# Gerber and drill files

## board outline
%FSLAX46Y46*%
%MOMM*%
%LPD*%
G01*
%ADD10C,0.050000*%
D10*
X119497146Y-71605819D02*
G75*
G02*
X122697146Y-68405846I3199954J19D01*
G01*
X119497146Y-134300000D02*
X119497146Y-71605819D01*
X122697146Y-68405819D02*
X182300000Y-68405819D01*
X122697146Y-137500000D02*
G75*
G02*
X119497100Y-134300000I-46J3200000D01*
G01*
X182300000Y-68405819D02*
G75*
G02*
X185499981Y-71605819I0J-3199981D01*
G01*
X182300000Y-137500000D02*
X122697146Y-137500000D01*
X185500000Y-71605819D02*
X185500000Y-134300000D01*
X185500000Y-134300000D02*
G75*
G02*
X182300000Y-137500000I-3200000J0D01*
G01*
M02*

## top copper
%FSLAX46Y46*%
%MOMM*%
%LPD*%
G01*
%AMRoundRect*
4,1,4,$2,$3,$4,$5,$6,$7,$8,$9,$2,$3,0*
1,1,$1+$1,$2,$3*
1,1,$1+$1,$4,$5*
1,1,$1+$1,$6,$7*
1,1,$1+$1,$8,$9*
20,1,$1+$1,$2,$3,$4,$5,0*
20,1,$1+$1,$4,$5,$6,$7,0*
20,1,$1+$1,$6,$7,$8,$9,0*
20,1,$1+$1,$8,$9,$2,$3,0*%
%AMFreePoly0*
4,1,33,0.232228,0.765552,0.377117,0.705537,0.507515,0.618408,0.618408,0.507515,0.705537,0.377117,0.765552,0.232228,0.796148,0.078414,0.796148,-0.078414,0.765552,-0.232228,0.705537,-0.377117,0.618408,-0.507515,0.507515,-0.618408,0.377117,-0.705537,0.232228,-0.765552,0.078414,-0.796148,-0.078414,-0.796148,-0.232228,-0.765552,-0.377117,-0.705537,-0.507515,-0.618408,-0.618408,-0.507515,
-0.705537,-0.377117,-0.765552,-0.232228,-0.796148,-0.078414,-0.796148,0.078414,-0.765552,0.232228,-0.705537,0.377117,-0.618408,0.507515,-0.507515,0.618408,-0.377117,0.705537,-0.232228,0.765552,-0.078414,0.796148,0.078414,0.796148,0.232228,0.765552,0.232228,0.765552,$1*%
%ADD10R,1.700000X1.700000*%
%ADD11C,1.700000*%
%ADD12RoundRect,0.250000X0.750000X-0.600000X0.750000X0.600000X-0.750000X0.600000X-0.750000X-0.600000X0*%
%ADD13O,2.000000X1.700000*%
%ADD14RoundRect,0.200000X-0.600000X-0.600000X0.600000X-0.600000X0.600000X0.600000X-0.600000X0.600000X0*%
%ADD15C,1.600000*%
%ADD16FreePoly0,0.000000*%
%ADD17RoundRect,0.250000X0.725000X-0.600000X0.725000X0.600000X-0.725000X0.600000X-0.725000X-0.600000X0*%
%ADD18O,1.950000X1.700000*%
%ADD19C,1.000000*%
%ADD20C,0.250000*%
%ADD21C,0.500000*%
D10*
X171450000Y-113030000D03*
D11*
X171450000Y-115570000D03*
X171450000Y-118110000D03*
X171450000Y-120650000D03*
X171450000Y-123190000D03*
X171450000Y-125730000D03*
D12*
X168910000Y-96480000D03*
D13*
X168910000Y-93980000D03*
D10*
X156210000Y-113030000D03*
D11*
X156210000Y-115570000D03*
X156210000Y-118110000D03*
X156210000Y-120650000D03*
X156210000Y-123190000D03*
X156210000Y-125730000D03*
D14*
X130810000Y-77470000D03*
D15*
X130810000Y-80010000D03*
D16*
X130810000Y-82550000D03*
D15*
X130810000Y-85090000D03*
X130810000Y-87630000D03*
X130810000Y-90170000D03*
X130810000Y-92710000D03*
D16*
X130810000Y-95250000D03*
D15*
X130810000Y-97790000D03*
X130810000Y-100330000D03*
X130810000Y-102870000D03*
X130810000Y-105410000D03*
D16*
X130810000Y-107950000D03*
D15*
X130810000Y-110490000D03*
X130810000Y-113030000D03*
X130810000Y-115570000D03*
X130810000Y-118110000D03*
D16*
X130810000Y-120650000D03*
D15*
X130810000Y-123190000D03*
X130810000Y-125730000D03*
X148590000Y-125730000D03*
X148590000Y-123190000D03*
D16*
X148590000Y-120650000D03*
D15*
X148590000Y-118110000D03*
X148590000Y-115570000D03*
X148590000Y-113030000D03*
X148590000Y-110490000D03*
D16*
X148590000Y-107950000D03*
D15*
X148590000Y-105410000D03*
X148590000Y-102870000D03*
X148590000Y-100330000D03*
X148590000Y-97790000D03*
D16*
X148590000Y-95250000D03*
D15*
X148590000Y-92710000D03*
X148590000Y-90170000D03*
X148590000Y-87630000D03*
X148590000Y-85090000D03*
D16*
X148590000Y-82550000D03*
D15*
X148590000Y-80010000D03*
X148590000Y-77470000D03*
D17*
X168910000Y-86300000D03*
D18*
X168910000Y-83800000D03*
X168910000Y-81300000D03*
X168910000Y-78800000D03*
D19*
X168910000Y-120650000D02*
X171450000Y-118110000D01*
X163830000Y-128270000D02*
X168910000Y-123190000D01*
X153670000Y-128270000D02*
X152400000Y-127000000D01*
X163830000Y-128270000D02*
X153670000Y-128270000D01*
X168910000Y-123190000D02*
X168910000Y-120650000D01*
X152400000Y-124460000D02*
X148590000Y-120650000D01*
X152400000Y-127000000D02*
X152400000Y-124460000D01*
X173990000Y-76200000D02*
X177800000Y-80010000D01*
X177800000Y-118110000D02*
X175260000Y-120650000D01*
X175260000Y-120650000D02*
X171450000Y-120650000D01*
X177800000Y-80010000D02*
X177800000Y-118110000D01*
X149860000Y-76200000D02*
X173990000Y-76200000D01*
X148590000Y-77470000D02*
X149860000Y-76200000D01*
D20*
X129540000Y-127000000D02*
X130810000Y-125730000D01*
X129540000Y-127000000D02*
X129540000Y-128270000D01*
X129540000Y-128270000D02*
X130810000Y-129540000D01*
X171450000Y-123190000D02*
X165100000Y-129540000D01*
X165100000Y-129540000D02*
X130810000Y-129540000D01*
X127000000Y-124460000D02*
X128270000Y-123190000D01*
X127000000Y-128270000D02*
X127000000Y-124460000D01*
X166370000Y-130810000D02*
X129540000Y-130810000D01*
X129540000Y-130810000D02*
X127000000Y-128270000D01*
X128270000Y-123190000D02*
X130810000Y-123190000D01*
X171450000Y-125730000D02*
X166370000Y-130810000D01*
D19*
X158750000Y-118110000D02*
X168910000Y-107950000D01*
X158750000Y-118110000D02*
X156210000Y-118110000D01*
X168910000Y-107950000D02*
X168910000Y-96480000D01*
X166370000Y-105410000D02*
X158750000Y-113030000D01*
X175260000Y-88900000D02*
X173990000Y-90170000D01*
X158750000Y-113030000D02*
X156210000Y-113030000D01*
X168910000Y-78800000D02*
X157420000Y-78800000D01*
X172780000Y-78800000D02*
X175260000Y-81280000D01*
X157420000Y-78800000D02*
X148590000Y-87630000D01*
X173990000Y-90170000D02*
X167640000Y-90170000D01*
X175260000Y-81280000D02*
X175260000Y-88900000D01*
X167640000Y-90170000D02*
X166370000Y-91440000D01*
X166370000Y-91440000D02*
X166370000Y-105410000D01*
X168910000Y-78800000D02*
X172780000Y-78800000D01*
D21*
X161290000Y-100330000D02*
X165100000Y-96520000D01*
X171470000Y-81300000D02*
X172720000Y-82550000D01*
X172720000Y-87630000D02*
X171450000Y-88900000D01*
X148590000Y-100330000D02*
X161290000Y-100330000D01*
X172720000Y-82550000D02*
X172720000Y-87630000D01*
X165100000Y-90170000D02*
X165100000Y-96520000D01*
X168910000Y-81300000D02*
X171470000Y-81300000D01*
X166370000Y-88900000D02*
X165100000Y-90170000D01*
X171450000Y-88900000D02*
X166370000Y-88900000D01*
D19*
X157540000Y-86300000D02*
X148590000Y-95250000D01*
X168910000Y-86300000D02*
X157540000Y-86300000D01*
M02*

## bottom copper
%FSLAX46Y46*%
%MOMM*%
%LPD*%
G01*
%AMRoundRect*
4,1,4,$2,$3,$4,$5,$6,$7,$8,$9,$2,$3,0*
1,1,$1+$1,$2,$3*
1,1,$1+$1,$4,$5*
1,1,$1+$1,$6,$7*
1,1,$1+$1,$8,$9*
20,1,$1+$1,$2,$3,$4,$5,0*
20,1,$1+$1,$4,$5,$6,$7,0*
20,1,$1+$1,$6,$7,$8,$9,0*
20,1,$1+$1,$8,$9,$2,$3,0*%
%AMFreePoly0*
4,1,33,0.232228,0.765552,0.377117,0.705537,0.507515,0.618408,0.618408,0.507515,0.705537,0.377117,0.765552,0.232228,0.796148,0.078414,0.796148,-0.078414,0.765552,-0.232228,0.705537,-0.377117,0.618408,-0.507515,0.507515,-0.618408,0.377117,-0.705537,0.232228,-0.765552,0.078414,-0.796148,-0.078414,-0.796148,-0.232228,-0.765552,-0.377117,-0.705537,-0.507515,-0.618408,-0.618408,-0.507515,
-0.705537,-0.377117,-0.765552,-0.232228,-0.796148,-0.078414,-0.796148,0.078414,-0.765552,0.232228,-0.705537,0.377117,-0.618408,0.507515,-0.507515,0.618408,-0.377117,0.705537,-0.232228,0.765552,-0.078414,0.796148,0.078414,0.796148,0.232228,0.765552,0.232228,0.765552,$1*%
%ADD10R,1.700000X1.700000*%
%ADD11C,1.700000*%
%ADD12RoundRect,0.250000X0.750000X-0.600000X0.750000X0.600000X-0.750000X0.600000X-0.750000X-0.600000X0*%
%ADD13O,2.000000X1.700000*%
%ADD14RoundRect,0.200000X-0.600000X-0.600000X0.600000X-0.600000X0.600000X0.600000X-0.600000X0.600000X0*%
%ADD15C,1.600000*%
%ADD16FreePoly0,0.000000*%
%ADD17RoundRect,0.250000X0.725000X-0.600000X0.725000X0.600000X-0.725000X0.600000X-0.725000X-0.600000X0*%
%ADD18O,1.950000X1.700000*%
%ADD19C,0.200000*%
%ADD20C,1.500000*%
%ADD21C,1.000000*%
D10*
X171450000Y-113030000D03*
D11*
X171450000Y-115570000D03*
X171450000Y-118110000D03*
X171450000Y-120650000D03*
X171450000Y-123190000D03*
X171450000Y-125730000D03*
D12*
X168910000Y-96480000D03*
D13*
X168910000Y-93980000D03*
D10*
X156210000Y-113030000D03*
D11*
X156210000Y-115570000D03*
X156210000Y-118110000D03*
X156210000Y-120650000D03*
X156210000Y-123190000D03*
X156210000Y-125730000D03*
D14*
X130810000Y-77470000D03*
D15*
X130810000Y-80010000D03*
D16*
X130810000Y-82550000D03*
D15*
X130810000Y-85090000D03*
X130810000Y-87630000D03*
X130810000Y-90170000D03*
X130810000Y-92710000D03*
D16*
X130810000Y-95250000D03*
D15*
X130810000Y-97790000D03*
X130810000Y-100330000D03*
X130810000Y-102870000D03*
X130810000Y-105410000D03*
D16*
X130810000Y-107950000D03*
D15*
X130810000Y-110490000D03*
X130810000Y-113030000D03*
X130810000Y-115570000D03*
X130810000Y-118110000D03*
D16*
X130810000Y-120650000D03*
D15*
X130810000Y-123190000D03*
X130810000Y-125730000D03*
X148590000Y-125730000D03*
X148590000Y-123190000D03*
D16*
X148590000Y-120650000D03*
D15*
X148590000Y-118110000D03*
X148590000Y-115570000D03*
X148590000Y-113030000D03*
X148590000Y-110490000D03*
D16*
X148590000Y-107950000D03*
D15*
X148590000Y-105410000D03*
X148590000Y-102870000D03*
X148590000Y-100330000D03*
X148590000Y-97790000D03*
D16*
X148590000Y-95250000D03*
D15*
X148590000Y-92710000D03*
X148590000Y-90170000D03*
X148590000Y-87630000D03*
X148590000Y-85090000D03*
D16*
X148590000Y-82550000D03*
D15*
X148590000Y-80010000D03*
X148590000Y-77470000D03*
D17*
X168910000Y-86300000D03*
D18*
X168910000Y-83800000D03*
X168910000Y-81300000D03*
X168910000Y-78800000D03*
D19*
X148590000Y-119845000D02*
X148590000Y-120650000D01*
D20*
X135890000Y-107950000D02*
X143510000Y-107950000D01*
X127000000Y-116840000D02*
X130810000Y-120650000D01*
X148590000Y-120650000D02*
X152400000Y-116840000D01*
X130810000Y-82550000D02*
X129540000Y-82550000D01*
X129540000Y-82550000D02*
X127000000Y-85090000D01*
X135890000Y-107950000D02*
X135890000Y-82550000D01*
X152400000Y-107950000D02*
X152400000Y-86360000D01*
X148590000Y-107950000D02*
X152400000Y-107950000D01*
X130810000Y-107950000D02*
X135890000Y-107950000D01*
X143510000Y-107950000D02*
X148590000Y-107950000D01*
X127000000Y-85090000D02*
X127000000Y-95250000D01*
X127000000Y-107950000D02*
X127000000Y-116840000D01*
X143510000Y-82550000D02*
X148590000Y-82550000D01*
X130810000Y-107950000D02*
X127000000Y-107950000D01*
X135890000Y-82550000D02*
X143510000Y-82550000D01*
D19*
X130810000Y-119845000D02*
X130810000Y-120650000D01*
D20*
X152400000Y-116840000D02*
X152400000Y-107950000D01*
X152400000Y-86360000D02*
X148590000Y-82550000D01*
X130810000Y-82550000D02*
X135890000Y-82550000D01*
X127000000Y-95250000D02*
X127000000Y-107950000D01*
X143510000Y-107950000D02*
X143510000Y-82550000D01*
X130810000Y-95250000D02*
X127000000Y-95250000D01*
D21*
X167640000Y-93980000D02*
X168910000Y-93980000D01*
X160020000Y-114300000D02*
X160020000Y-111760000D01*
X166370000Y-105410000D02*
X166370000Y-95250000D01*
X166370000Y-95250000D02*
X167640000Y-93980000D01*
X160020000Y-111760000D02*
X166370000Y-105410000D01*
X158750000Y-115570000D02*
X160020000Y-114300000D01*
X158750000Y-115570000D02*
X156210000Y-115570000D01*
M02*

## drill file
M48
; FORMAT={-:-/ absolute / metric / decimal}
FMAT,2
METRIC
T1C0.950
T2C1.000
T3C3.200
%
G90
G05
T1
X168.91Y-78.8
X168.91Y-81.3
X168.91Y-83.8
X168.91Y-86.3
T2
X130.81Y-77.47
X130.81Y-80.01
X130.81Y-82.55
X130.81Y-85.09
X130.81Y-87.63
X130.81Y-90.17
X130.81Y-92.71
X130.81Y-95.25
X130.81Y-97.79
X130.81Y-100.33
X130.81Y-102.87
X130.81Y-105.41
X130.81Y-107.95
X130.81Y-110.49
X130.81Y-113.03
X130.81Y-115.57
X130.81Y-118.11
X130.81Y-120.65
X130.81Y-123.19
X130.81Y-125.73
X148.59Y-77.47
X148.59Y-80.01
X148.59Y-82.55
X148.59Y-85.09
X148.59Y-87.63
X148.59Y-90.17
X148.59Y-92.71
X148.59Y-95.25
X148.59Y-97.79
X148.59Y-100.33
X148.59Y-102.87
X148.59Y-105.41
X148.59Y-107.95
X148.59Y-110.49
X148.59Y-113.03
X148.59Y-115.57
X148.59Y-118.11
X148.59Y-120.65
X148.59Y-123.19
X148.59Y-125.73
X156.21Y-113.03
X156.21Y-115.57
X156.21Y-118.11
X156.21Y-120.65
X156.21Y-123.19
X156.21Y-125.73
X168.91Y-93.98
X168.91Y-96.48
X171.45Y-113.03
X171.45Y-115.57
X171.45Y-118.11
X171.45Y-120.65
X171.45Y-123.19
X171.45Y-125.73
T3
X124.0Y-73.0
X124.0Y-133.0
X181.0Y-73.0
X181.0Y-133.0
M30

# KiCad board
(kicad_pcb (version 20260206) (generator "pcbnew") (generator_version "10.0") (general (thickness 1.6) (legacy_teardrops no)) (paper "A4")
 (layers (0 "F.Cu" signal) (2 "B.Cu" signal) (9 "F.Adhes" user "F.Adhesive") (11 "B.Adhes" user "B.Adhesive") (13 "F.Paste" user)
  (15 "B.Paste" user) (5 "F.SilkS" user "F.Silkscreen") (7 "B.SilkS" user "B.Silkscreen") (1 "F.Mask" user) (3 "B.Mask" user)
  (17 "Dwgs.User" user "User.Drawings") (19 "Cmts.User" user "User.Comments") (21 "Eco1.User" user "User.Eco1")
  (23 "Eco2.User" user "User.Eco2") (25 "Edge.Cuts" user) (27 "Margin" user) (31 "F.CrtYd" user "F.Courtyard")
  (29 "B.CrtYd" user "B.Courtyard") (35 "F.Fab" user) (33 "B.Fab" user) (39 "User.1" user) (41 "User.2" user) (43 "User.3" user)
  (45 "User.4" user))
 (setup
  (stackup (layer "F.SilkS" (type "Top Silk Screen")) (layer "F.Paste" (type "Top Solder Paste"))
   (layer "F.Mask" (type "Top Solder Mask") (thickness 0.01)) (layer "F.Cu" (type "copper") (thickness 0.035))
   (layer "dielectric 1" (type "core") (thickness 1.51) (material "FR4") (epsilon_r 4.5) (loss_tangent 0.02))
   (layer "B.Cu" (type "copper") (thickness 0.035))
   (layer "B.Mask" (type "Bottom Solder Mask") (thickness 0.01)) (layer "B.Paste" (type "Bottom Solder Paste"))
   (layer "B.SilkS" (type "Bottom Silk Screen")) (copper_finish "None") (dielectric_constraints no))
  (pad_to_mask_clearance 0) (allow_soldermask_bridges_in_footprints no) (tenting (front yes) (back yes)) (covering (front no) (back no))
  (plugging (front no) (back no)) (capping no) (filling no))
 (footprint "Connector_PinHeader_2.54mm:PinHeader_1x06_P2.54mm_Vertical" (layer "F.Cu") (at 171.45 113.03)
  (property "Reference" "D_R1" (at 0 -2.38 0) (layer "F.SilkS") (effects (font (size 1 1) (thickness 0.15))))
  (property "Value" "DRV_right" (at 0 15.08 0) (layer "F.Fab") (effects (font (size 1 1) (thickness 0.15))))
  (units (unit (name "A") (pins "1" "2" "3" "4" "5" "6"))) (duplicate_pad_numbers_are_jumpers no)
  (pad "1" thru_hole rect (at 0 0) (size 1.7 1.7) (drill 1) (layers "*.Cu" "*.Mask") (remove_unused_layers no) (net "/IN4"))
  (pad "2" thru_hole circle (at 0 2.54) (size 1.7 1.7) (drill 1) (layers "*.Cu" "*.Mask") (remove_unused_layers no) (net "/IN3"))
  (pad "3" thru_hole circle (at 0 5.08) (size 1.7 1.7) (drill 1) (layers "*.Cu" "*.Mask") (remove_unused_layers no) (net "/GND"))
  (pad "4" thru_hole circle (at 0 7.62) (size 1.7 1.7) (drill 1) (layers "*.Cu" "*.Mask") (remove_unused_layers no) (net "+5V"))
  (pad "5" thru_hole circle (at 0 10.16) (size 1.7 1.7) (drill 1) (layers "*.Cu" "*.Mask") (remove_unused_layers no) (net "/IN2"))
  (pad "6" thru_hole circle (at 0 12.7) (size 1.7 1.7) (drill 1) (layers "*.Cu" "*.Mask") (remove_unused_layers no) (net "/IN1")))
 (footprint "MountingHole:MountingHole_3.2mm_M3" (layer "F.Cu") (at 181 133)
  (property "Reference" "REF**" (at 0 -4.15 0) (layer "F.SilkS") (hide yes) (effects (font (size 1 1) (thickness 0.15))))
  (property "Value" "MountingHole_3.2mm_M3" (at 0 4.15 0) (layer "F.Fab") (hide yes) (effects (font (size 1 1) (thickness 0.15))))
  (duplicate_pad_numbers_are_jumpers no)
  (pad "" np_thru_hole circle (at 0 0) (size 3.2 3.2) (drill 3.2) (layers "*.Cu" "*.Mask")))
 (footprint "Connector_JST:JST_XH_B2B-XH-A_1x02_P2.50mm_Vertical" (layer "F.Cu") (at 168.91 96.48 90)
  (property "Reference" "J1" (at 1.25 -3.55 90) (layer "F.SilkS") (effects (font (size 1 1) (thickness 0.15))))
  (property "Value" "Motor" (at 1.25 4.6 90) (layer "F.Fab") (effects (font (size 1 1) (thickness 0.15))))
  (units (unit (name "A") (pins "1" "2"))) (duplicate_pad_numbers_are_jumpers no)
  (pad "1" thru_hole roundrect (at 0 0 90) (size 1.7 2) (drill 1) (layers "*.Cu" "*.Mask") (remove_unused_layers no)
   (roundrect_rratio 0.147059) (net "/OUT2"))
  (pad "2" thru_hole oval (at 2.5 0 90) (size 1.7 2) (drill 1) (layers "*.Cu" "*.Mask") (remove_unused_layers no) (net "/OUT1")))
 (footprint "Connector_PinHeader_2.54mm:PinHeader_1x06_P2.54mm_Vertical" (layer "F.Cu") (at 156.21 113.03)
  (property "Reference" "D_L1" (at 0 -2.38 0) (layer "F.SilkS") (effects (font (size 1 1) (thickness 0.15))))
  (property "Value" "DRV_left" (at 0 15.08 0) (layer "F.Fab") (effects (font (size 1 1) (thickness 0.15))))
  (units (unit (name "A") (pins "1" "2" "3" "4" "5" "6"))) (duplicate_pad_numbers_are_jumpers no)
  (pad "1" thru_hole rect (at 0 0) (size 1.7 1.7) (drill 1) (layers "*.Cu" "*.Mask") (remove_unused_layers no) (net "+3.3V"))
  (pad "2" thru_hole circle (at 0 2.54) (size 1.7 1.7) (drill 1) (layers "*.Cu" "*.Mask") (remove_unused_layers no) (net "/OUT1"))
  (pad "3" thru_hole circle (at 0 5.08) (size 1.7 1.7) (drill 1) (layers "*.Cu" "*.Mask") (remove_unused_layers no) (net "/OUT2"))
  (pad "4" thru_hole circle (at 0 7.62) (size 1.7 1.7) (drill 1) (layers "*.Cu" "*.Mask") (remove_unused_layers no) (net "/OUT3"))
  (pad "5" thru_hole circle (at 0 10.16) (size 1.7 1.7) (drill 1) (layers "*.Cu" "*.Mask") (remove_unused_layers no) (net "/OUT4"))
  (pad "6" thru_hole circle (at 0 12.7) (size 1.7 1.7) (drill 1) (layers "*.Cu" "*.Mask") (remove_unused_layers no) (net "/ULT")))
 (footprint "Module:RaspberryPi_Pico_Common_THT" (layer "F.Cu") (at 130.81 77.47)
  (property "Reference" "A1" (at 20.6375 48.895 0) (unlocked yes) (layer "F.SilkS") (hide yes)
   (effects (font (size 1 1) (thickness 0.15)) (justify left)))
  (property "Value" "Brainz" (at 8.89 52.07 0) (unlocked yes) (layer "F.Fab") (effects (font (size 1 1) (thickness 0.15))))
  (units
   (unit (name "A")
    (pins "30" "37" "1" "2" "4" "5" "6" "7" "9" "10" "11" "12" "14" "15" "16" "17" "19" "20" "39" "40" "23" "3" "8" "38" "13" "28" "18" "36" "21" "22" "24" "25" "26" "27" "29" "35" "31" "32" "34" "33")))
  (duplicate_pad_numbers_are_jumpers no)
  (pad "1" thru_hole roundrect (at 0 0) (size 1.6 1.6) (drill 1) (layers "*.Cu" "*.Mask") (remove_unused_layers no) (roundrect_rratio 0.125)
   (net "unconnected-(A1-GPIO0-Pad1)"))
  (pad "2" thru_hole circle (at 0 2.54) (size 1.6 1.6) (drill 1) (layers "*.Cu" "*.Mask") (remove_unused_layers no)
   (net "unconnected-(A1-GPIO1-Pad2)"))
  (pad "3" thru_hole custom (at 0 5.08) (size 1.6 1.6) (drill 1) (layers "*.Cu" "*.Mask") (remove_unused_layers no) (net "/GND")
   (options (clearance outline) (anchor circle)) (primitives))
  (pad "4" thru_hole circle (at 0 7.62) (size 1.6 1.6) (drill 1) (layers "*.Cu" "*.Mask") (remove_unused_layers no)
   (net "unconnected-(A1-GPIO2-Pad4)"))
  (pad "5" thru_hole circle (at 0 10.16) (size 1.6 1.6) (drill 1) (layers "*.Cu" "*.Mask") (remove_unused_layers no)
   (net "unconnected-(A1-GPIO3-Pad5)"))
  (pad "6" thru_hole circle (at 0 12.7) (size 1.6 1.6) (drill 1) (layers "*.Cu" "*.Mask") (remove_unused_layers no)
   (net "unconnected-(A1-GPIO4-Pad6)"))
  (pad "7" thru_hole circle (at 0 15.24) (size 1.6 1.6) (drill 1) (layers "*.Cu" "*.Mask") (remove_unused_layers no)
   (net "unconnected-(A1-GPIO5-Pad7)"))
  (pad "8" thru_hole custom (at 0 17.78) (size 1.6 1.6) (drill 1) (layers "*.Cu" "*.Mask") (remove_unused_layers no) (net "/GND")
   (options (clearance outline) (anchor circle)) (primitives))
  (pad "9" thru_hole circle (at 0 20.32) (size 1.6 1.6) (drill 1) (layers "*.Cu" "*.Mask") (remove_unused_layers no)
   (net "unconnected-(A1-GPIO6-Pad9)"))
  (pad "10" thru_hole circle (at 0 22.86) (size 1.6 1.6) (drill 1) (layers "*.Cu" "*.Mask") (remove_unused_layers no)
   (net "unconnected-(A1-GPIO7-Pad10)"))
  (pad "11" thru_hole circle (at 0 25.4) (size 1.6 1.6) (drill 1) (layers "*.Cu" "*.Mask") (remove_unused_layers no)
   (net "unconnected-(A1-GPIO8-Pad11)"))
  (pad "12" thru_hole circle (at 0 27.94) (size 1.6 1.6) (drill 1) (layers "*.Cu" "*.Mask") (remove_unused_layers no)
   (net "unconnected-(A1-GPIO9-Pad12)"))
  (pad "13" thru_hole custom (at 0 30.48) (size 1.6 1.6) (drill 1) (layers "*.Cu" "*.Mask") (remove_unused_layers no) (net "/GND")
   (options (clearance outline) (anchor circle)) (primitives))
  (pad "14" thru_hole circle (at 0 33.02) (size 1.6 1.6) (drill 1) (layers "*.Cu" "*.Mask") (remove_unused_layers no)
   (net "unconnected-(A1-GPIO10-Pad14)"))
  (pad "15" thru_hole circle (at 0 35.56) (size 1.6 1.6) (drill 1) (layers "*.Cu" "*.Mask") (remove_unused_layers no)
   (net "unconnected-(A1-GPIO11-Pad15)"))
  (pad "16" thru_hole circle (at 0 38.1) (size 1.6 1.6) (drill 1) (layers "*.Cu" "*.Mask") (remove_unused_layers no)
   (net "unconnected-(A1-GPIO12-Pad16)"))
  (pad "17" thru_hole circle (at 0 40.64) (size 1.6 1.6) (drill 1) (layers "*.Cu" "*.Mask") (remove_unused_layers no)
   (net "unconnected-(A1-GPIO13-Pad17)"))
  (pad "18" thru_hole custom (at 0 43.18) (size 1.6 1.6) (drill 1) (layers "*.Cu" "*.Mask") (remove_unused_layers no) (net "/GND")
   (options (clearance outline) (anchor circle)) (primitives))
  (pad "19" thru_hole circle (at 0 45.72) (size 1.6 1.6) (drill 1) (layers "*.Cu" "*.Mask") (remove_unused_layers no) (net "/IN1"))
  (pad "20" thru_hole circle (at 0 48.26) (size 1.6 1.6) (drill 1) (layers "*.Cu" "*.Mask") (remove_unused_layers no) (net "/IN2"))
  (pad "21" thru_hole circle (at 17.78 48.26) (size 1.6 1.6) (drill 1) (layers "*.Cu" "*.Mask") (remove_unused_layers no)
   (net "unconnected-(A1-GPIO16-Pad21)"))
  (pad "22" thru_hole circle (at 17.78 45.72) (size 1.6 1.6) (drill 1) (layers "*.Cu" "*.Mask") (remove_unused_layers no)
   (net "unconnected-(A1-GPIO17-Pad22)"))
  (pad "23" thru_hole custom (at 17.78 43.18) (size 1.6 1.6) (drill 1) (layers "*.Cu" "*.Mask") (remove_unused_layers no) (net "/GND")
   (options (clearance outline) (anchor circle)) (primitives))
  (pad "24" thru_hole circle (at 17.78 40.64) (size 1.6 1.6) (drill 1) (layers "*.Cu" "*.Mask") (remove_unused_layers no)
   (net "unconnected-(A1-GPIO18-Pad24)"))
  (pad "25" thru_hole circle (at 17.78 38.1) (size 1.6 1.6) (drill 1) (layers "*.Cu" "*.Mask") (remove_unused_layers no)
   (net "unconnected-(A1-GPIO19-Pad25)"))
  (pad "26" thru_hole circle (at 17.78 35.56) (size 1.6 1.6) (drill 1) (layers "*.Cu" "*.Mask") (remove_unused_layers no)
   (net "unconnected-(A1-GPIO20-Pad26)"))
  (pad "27" thru_hole circle (at 17.78 33.02) (size 1.6 1.6) (drill 1) (layers "*.Cu" "*.Mask") (remove_unused_layers no)
   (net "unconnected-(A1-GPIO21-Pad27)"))
  (pad "28" thru_hole custom (at 17.78 30.48) (size 1.6 1.6) (drill 1) (layers "*.Cu" "*.Mask") (remove_unused_layers no) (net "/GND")
   (options (clearance outline) (anchor circle)) (primitives))
  (pad "29" thru_hole circle (at 17.78 27.94) (size 1.6 1.6) (drill 1) (layers "*.Cu" "*.Mask") (remove_unused_layers no)
   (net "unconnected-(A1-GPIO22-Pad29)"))
  (pad "30" thru_hole circle (at 17.78 25.4) (size 1.6 1.6) (drill 1) (layers "*.Cu" "*.Mask") (remove_unused_layers no)
   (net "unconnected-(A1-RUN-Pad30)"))
  (pad "31" thru_hole circle (at 17.78 22.86) (size 1.6 1.6) (drill 1) (layers "*.Cu" "*.Mask") (remove_unused_layers no) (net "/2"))
  (pad "32" thru_hole circle (at 17.78 20.32) (size 1.6 1.6) (drill 1) (layers "*.Cu" "*.Mask") (remove_unused_layers no)
   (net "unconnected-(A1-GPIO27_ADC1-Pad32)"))
  (pad "33" thru_hole custom (at 17.78 17.78) (size 1.6 1.6) (drill 1) (layers "*.Cu" "*.Mask") (remove_unused_layers no) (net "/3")
   (options (clearance outline) (anchor circle)) (primitives))
  (pad "34" thru_hole circle (at 17.78 15.24) (size 1.6 1.6) (drill 1) (layers "*.Cu" "*.Mask") (remove_unused_layers no)
   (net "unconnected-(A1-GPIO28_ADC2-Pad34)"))
  (pad "35" thru_hole circle (at 17.78 12.7) (size 1.6 1.6) (drill 1) (layers "*.Cu" "*.Mask") (remove_unused_layers no)
   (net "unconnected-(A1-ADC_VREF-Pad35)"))
  (pad "36" thru_hole circle (at 17.78 10.16) (size 1.6 1.6) (drill 1) (layers "*.Cu" "*.Mask") (remove_unused_layers no) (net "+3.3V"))
  (pad "37" thru_hole circle (at 17.78 7.62) (size 1.6 1.6) (drill 1) (layers "*.Cu" "*.Mask") (remove_unused_layers no)
   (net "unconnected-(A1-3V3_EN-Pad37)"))
  (pad "38" thru_hole custom (at 17.78 5.08) (size 1.6 1.6) (drill 1) (layers "*.Cu" "*.Mask") (remove_unused_layers no) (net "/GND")
   (options (clearance outline) (anchor circle)) (primitives))
  (pad "39" thru_hole circle (at 17.78 2.54) (size 1.6 1.6) (drill 1) (layers "*.Cu" "*.Mask") (remove_unused_layers no)
   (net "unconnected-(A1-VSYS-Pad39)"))
  (pad "40" thru_hole circle (at 17.78 0) (size 1.6 1.6) (drill 1) (layers "*.Cu" "*.Mask") (remove_unused_layers no) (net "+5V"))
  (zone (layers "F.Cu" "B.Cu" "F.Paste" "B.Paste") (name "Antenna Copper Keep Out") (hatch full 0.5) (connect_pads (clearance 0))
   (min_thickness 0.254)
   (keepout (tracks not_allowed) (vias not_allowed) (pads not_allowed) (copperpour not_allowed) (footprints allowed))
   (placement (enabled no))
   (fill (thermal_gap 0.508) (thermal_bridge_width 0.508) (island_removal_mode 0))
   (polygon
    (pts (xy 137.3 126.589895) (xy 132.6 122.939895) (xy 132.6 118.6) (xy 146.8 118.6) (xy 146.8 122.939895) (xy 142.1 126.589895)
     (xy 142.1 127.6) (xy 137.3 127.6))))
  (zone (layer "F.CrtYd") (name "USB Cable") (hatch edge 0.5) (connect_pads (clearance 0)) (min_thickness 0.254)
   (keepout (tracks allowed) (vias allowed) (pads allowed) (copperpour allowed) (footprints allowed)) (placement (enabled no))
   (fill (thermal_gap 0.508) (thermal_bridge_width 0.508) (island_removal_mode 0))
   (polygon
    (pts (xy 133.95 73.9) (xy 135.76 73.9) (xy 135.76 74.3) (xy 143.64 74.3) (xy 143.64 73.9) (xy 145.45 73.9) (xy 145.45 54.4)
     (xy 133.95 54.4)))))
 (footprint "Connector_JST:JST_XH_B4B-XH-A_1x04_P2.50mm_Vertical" (layer "F.Cu") (at 168.91 86.3 90)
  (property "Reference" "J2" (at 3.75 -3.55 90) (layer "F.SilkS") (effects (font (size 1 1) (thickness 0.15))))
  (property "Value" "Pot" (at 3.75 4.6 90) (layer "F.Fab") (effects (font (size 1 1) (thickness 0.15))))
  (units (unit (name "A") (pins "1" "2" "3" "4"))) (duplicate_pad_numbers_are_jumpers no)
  (pad "1" thru_hole roundrect (at 0 0 90) (size 1.7 1.95) (drill 0.95) (layers "*.Cu" "*.Mask") (remove_unused_layers no)
   (roundrect_rratio 0.147059) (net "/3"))
  (pad "2" thru_hole oval (at 2.5 0 90) (size 1.7 1.95) (drill 0.95) (layers "*.Cu" "*.Mask") (remove_unused_layers no) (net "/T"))
  (pad "3" thru_hole oval (at 5 0 90) (size 1.7 1.95) (drill 0.95) (layers "*.Cu" "*.Mask") (remove_unused_layers no) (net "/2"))
  (pad "4" thru_hole oval (at 7.5 0 90) (size 1.7 1.95) (drill 0.95) (layers "*.Cu" "*.Mask") (remove_unused_layers no) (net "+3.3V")))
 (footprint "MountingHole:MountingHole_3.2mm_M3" (layer "F.Cu") (at 124 133)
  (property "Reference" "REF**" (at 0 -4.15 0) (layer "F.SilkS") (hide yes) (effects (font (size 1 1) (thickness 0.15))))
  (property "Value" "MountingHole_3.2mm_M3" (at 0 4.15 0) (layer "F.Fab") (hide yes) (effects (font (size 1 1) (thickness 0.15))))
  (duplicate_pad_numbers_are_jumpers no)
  (pad "" np_thru_hole circle (at 0 0) (size 3.2 3.2) (drill 3.2) (layers "*.Cu" "*.Mask")))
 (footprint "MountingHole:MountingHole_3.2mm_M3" (layer "F.Cu") (at 124 73)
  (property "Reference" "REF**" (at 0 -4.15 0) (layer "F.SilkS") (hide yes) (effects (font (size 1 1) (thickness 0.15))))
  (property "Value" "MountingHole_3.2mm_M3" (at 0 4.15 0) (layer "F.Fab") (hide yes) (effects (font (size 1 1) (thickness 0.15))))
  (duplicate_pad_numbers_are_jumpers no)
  (pad "" np_thru_hole circle (at 0 0) (size 3.2 3.2) (drill 3.2) (layers "*.Cu" "*.Mask")))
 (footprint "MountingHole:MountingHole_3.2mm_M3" (layer "F.Cu") (at 181 73)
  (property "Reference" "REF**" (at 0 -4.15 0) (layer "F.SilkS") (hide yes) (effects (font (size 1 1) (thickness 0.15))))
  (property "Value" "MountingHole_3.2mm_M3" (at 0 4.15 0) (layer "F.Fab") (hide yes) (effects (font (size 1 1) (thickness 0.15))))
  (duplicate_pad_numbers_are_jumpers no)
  (pad "" np_thru_hole circle (at 0 0) (size 3.2 3.2) (drill 3.2) (layers "*.Cu" "*.Mask")))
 (gr_arc (start 119.497146 71.605819) (mid 120.434404 69.343077) (end 122.697146 68.405819) (stroke (width 0.05) (type default))
  (layer "Edge.Cuts"))
 (gr_line (start 119.497146 134.3) (end 119.497146 71.605819) (stroke (width 0.05) (type default)) (layer "Edge.Cuts"))
 (gr_line (start 122.697146 68.405819) (end 182.3 68.405819) (stroke (width 0.05) (type default)) (layer "Edge.Cuts"))
 (gr_arc (start 122.697146 137.5) (mid 120.434404 136.562742) (end 119.497146 134.3) (stroke (width 0.05) (type default))
  (layer "Edge.Cuts"))
 (gr_arc (start 182.3 68.405819) (mid 184.562735 69.343078) (end 185.5 71.605819) (stroke (width 0.05) (type default)) (layer "Edge.Cuts"))
 (gr_line (start 182.3 137.5) (end 122.697146 137.5) (stroke (width 0.05) (type default)) (layer "Edge.Cuts"))
 (gr_line (start 185.5 71.605819) (end 185.5 134.3) (stroke (width 0.05) (type default)) (layer "Edge.Cuts"))
 (gr_arc (start 185.5 134.3) (mid 184.562742 136.562742) (end 182.3 137.5) (stroke (width 0.05) (type default)) (layer "Edge.Cuts"))
 (segment (start 168.91 120.65) (end 171.45 118.11) (width 1) (layer "F.Cu") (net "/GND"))
 (segment (start 163.83 128.27) (end 168.91 123.19) (width 1) (layer "F.Cu") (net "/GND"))
 (segment (start 153.67 128.27) (end 152.4 127) (width 1) (layer "F.Cu") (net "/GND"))
 (segment (start 163.83 128.27) (end 153.67 128.27) (width 1) (layer "F.Cu") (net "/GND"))
 (segment (start 168.91 123.19) (end 168.91 120.65) (width 1) (layer "F.Cu") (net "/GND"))
 (segment (start 152.4 124.46) (end 148.59 120.65) (width 1) (layer "F.Cu") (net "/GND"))
 (segment (start 152.4 127) (end 152.4 124.46) (width 1) (layer "F.Cu") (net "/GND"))
 (segment (start 148.59 119.845) (end 148.59 120.65) (width 0.2) (layer "B.Cu") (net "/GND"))
 (segment (start 135.89 107.95) (end 143.51 107.95) (width 1.5) (layer "B.Cu") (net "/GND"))
 (segment (start 127 116.84) (end 130.81 120.65) (width 1.5) (layer "B.Cu") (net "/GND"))
 (segment (start 148.59 120.65) (end 152.4 116.84) (width 1.5) (layer "B.Cu") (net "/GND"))
 (segment (start 130.81 82.55) (end 129.54 82.55) (width 1.5) (layer "B.Cu") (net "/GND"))
 (segment (start 129.54 82.55) (end 127 85.09) (width 1.5) (layer "B.Cu") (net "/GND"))
 (segment (start 135.89 107.95) (end 135.89 82.55) (width 1.5) (layer "B.Cu") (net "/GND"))
 (segment (start 152.4 107.95) (end 152.4 86.36) (width 1.5) (layer "B.Cu") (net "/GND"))
 (segment (start 148.59 107.95) (end 152.4 107.95) (width 1.5) (layer "B.Cu") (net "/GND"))
 (segment (start 130.81 107.95) (end 135.89 107.95) (width 1.5) (layer "B.Cu") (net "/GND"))
 (segment (start 143.51 107.95) (end 148.59 107.95) (width 1.5) (layer "B.Cu") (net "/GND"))
 (segment (start 127 85.09) (end 127 95.25) (width 1.5) (layer "B.Cu") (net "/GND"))
 (segment (start 127 107.95) (end 127 116.84) (width 1.5) (layer "B.Cu") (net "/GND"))
 (segment (start 143.51 82.55) (end 148.59 82.55) (width 1.5) (layer "B.Cu") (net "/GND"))
 (segment (start 130.81 107.95) (end 127 107.95) (width 1.5) (layer "B.Cu") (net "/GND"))
 (segment (start 135.89 82.55) (end 143.51 82.55) (width 1.5) (layer "B.Cu") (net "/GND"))
 (segment (start 130.81 119.845) (end 130.81 120.65) (width 0.2) (layer "B.Cu") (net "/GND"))
 (segment (start 152.4 116.84) (end 152.4 107.95) (width 1.5) (layer "B.Cu") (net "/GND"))
 (segment (start 152.4 86.36) (end 148.59 82.55) (width 1.5) (layer "B.Cu") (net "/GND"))
 (segment (start 130.81 82.55) (end 135.89 82.55) (width 1.5) (layer "B.Cu") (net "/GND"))
 (segment (start 127 95.25) (end 127 107.95) (width 1.5) (layer "B.Cu") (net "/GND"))
 (segment (start 143.51 107.95) (end 143.51 82.55) (width 1.5) (layer "B.Cu") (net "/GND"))
 (segment (start 130.81 95.25) (end 127 95.25) (width 1.5) (layer "B.Cu") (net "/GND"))
 (segment (start 173.99 76.2) (end 177.8 80.01) (width 1) (layer "F.Cu") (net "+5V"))
 (segment (start 177.8 118.11) (end 175.26 120.65) (width 1) (layer "F.Cu") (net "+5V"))
 (segment (start 175.26 120.65) (end 171.45 120.65) (width 1) (layer "F.Cu") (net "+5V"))
 (segment (start 177.8 80.01) (end 177.8 118.11) (width 1) (layer "F.Cu") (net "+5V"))
 (segment (start 149.86 76.2) (end 173.99 76.2) (width 1) (layer "F.Cu") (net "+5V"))
 (segment (start 148.59 77.47) (end 149.86 76.2) (width 1) (layer "F.Cu") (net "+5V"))
 (segment (start 129.54 127) (end 130.81 125.73) (width 0.25) (layer "F.Cu") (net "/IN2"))
 (segment (start 129.54 127) (end 129.54 128.27) (width 0.25) (layer "F.Cu") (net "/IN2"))
 (segment (start 129.54 128.27) (end 130.81 129.54) (width 0.25) (layer "F.Cu") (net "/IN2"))
 (segment (start 171.45 123.19) (end 165.1 129.54) (width 0.25) (layer "F.Cu") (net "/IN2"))
 (segment (start 165.1 129.54) (end 130.81 129.54) (width 0.25) (layer "F.Cu") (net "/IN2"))
 (segment (start 127 124.46) (end 128.27 123.19) (width 0.25) (layer "F.Cu") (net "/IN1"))
 (segment (start 127 128.27) (end 127 124.46) (width 0.25) (layer "F.Cu") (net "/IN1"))
 (segment (start 166.37 130.81) (end 129.54 130.81) (width 0.25) (layer "F.Cu") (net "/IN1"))
 (segment (start 129.54 130.81) (end 127 128.27) (width 0.25) (layer "F.Cu") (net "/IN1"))
 (segment (start 128.27 123.19) (end 130.81 123.19) (width 0.25) (layer "F.Cu") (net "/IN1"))
 (segment (start 171.45 125.73) (end 166.37 130.81) (width 0.25) (layer "F.Cu") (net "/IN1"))
 (segment (start 158.75 118.11) (end 168.91 107.95) (width 1) (layer "F.Cu") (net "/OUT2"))
 (segment (start 158.75 118.11) (end 156.21 118.11) (width 1) (layer "F.Cu") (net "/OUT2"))
 (segment (start 168.91 107.95) (end 168.91 96.48) (width 1) (layer "F.Cu") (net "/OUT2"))
 (segment (start 167.64 93.98) (end 168.91 93.98) (width 1) (layer "B.Cu") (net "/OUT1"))
 (segment (start 160.02 114.3) (end 160.02 111.76) (width 1) (layer "B.Cu") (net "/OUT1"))
 (segment (start 166.37 105.41) (end 166.37 95.25) (width 1) (layer "B.Cu") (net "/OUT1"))
 (segment (start 166.37 95.25) (end 167.64 93.98) (width 1) (layer "B.Cu") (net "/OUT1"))
 (segment (start 160.02 111.76) (end 166.37 105.41) (width 1) (layer "B.Cu") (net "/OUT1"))
 (segment (start 158.75 115.57) (end 160.02 114.3) (width 1) (layer "B.Cu") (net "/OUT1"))
 (segment (start 158.75 115.57) (end 156.21 115.57) (width 1) (layer "B.Cu") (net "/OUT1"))
 (segment (start 166.37 105.41) (end 158.75 113.03) (width 1) (layer "F.Cu") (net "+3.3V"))
 (segment (start 175.26 88.9) (end 173.99 90.17) (width 1) (layer "F.Cu") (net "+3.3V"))
 (segment (start 158.75 113.03) (end 156.21 113.03) (width 1) (layer "F.Cu") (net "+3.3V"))
 (segment (start 168.91 78.8) (end 157.42 78.8) (width 1) (layer "F.Cu") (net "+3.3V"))
 (segment (start 172.78 78.8) (end 175.26 81.28) (width 1) (layer "F.Cu") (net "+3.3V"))
 (segment (start 157.42 78.8) (end 148.59 87.63) (width 1) (layer "F.Cu") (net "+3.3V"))
 (segment (start 173.99 90.17) (end 167.64 90.17) (width 1) (layer "F.Cu") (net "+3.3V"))
 (segment (start 175.26 81.28) (end 175.26 88.9) (width 1) (layer "F.Cu") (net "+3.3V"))
 (segment (start 167.64 90.17) (end 166.37 91.44) (width 1) (layer "F.Cu") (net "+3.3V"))
 (segment (start 166.37 91.44) (end 166.37 105.41) (width 1) (layer "F.Cu") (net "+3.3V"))
 (segment (start 168.91 78.8) (end 172.78 78.8) (width 1) (layer "F.Cu") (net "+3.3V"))
 (segment (start 161.29 100.33) (end 165.1 96.52) (width 0.5) (layer "F.Cu") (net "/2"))
 (segment (start 171.47 81.3) (end 172.72 82.55) (width 0.5) (layer "F.Cu") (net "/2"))
 (segment (start 172.72 87.63) (end 171.45 88.9) (width 0.5) (layer "F.Cu") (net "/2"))
 (segment (start 148.59 100.33) (end 161.29 100.33) (width 0.5) (layer "F.Cu") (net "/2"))
 (segment (start 172.72 82.55) (end 172.72 87.63) (width 0.5) (layer "F.Cu") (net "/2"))
 (segment (start 165.1 90.17) (end 165.1 96.52) (width 0.5) (layer "F.Cu") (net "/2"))
 (segment (start 168.91 81.3) (end 171.47 81.3) (width 0.5) (layer "F.Cu") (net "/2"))
 (segment (start 166.37 88.9) (end 165.1 90.17) (width 0.5) (layer "F.Cu") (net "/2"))
 (segment (start 171.45 88.9) (end 166.37 88.9) (width 0.5) (layer "F.Cu") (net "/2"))
 (segment (start 157.54 86.3) (end 148.59 95.25) (width 1) (layer "F.Cu") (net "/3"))
 (segment (start 168.91 86.3) (end 157.54 86.3) (width 1) (layer "F.Cu") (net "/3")))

